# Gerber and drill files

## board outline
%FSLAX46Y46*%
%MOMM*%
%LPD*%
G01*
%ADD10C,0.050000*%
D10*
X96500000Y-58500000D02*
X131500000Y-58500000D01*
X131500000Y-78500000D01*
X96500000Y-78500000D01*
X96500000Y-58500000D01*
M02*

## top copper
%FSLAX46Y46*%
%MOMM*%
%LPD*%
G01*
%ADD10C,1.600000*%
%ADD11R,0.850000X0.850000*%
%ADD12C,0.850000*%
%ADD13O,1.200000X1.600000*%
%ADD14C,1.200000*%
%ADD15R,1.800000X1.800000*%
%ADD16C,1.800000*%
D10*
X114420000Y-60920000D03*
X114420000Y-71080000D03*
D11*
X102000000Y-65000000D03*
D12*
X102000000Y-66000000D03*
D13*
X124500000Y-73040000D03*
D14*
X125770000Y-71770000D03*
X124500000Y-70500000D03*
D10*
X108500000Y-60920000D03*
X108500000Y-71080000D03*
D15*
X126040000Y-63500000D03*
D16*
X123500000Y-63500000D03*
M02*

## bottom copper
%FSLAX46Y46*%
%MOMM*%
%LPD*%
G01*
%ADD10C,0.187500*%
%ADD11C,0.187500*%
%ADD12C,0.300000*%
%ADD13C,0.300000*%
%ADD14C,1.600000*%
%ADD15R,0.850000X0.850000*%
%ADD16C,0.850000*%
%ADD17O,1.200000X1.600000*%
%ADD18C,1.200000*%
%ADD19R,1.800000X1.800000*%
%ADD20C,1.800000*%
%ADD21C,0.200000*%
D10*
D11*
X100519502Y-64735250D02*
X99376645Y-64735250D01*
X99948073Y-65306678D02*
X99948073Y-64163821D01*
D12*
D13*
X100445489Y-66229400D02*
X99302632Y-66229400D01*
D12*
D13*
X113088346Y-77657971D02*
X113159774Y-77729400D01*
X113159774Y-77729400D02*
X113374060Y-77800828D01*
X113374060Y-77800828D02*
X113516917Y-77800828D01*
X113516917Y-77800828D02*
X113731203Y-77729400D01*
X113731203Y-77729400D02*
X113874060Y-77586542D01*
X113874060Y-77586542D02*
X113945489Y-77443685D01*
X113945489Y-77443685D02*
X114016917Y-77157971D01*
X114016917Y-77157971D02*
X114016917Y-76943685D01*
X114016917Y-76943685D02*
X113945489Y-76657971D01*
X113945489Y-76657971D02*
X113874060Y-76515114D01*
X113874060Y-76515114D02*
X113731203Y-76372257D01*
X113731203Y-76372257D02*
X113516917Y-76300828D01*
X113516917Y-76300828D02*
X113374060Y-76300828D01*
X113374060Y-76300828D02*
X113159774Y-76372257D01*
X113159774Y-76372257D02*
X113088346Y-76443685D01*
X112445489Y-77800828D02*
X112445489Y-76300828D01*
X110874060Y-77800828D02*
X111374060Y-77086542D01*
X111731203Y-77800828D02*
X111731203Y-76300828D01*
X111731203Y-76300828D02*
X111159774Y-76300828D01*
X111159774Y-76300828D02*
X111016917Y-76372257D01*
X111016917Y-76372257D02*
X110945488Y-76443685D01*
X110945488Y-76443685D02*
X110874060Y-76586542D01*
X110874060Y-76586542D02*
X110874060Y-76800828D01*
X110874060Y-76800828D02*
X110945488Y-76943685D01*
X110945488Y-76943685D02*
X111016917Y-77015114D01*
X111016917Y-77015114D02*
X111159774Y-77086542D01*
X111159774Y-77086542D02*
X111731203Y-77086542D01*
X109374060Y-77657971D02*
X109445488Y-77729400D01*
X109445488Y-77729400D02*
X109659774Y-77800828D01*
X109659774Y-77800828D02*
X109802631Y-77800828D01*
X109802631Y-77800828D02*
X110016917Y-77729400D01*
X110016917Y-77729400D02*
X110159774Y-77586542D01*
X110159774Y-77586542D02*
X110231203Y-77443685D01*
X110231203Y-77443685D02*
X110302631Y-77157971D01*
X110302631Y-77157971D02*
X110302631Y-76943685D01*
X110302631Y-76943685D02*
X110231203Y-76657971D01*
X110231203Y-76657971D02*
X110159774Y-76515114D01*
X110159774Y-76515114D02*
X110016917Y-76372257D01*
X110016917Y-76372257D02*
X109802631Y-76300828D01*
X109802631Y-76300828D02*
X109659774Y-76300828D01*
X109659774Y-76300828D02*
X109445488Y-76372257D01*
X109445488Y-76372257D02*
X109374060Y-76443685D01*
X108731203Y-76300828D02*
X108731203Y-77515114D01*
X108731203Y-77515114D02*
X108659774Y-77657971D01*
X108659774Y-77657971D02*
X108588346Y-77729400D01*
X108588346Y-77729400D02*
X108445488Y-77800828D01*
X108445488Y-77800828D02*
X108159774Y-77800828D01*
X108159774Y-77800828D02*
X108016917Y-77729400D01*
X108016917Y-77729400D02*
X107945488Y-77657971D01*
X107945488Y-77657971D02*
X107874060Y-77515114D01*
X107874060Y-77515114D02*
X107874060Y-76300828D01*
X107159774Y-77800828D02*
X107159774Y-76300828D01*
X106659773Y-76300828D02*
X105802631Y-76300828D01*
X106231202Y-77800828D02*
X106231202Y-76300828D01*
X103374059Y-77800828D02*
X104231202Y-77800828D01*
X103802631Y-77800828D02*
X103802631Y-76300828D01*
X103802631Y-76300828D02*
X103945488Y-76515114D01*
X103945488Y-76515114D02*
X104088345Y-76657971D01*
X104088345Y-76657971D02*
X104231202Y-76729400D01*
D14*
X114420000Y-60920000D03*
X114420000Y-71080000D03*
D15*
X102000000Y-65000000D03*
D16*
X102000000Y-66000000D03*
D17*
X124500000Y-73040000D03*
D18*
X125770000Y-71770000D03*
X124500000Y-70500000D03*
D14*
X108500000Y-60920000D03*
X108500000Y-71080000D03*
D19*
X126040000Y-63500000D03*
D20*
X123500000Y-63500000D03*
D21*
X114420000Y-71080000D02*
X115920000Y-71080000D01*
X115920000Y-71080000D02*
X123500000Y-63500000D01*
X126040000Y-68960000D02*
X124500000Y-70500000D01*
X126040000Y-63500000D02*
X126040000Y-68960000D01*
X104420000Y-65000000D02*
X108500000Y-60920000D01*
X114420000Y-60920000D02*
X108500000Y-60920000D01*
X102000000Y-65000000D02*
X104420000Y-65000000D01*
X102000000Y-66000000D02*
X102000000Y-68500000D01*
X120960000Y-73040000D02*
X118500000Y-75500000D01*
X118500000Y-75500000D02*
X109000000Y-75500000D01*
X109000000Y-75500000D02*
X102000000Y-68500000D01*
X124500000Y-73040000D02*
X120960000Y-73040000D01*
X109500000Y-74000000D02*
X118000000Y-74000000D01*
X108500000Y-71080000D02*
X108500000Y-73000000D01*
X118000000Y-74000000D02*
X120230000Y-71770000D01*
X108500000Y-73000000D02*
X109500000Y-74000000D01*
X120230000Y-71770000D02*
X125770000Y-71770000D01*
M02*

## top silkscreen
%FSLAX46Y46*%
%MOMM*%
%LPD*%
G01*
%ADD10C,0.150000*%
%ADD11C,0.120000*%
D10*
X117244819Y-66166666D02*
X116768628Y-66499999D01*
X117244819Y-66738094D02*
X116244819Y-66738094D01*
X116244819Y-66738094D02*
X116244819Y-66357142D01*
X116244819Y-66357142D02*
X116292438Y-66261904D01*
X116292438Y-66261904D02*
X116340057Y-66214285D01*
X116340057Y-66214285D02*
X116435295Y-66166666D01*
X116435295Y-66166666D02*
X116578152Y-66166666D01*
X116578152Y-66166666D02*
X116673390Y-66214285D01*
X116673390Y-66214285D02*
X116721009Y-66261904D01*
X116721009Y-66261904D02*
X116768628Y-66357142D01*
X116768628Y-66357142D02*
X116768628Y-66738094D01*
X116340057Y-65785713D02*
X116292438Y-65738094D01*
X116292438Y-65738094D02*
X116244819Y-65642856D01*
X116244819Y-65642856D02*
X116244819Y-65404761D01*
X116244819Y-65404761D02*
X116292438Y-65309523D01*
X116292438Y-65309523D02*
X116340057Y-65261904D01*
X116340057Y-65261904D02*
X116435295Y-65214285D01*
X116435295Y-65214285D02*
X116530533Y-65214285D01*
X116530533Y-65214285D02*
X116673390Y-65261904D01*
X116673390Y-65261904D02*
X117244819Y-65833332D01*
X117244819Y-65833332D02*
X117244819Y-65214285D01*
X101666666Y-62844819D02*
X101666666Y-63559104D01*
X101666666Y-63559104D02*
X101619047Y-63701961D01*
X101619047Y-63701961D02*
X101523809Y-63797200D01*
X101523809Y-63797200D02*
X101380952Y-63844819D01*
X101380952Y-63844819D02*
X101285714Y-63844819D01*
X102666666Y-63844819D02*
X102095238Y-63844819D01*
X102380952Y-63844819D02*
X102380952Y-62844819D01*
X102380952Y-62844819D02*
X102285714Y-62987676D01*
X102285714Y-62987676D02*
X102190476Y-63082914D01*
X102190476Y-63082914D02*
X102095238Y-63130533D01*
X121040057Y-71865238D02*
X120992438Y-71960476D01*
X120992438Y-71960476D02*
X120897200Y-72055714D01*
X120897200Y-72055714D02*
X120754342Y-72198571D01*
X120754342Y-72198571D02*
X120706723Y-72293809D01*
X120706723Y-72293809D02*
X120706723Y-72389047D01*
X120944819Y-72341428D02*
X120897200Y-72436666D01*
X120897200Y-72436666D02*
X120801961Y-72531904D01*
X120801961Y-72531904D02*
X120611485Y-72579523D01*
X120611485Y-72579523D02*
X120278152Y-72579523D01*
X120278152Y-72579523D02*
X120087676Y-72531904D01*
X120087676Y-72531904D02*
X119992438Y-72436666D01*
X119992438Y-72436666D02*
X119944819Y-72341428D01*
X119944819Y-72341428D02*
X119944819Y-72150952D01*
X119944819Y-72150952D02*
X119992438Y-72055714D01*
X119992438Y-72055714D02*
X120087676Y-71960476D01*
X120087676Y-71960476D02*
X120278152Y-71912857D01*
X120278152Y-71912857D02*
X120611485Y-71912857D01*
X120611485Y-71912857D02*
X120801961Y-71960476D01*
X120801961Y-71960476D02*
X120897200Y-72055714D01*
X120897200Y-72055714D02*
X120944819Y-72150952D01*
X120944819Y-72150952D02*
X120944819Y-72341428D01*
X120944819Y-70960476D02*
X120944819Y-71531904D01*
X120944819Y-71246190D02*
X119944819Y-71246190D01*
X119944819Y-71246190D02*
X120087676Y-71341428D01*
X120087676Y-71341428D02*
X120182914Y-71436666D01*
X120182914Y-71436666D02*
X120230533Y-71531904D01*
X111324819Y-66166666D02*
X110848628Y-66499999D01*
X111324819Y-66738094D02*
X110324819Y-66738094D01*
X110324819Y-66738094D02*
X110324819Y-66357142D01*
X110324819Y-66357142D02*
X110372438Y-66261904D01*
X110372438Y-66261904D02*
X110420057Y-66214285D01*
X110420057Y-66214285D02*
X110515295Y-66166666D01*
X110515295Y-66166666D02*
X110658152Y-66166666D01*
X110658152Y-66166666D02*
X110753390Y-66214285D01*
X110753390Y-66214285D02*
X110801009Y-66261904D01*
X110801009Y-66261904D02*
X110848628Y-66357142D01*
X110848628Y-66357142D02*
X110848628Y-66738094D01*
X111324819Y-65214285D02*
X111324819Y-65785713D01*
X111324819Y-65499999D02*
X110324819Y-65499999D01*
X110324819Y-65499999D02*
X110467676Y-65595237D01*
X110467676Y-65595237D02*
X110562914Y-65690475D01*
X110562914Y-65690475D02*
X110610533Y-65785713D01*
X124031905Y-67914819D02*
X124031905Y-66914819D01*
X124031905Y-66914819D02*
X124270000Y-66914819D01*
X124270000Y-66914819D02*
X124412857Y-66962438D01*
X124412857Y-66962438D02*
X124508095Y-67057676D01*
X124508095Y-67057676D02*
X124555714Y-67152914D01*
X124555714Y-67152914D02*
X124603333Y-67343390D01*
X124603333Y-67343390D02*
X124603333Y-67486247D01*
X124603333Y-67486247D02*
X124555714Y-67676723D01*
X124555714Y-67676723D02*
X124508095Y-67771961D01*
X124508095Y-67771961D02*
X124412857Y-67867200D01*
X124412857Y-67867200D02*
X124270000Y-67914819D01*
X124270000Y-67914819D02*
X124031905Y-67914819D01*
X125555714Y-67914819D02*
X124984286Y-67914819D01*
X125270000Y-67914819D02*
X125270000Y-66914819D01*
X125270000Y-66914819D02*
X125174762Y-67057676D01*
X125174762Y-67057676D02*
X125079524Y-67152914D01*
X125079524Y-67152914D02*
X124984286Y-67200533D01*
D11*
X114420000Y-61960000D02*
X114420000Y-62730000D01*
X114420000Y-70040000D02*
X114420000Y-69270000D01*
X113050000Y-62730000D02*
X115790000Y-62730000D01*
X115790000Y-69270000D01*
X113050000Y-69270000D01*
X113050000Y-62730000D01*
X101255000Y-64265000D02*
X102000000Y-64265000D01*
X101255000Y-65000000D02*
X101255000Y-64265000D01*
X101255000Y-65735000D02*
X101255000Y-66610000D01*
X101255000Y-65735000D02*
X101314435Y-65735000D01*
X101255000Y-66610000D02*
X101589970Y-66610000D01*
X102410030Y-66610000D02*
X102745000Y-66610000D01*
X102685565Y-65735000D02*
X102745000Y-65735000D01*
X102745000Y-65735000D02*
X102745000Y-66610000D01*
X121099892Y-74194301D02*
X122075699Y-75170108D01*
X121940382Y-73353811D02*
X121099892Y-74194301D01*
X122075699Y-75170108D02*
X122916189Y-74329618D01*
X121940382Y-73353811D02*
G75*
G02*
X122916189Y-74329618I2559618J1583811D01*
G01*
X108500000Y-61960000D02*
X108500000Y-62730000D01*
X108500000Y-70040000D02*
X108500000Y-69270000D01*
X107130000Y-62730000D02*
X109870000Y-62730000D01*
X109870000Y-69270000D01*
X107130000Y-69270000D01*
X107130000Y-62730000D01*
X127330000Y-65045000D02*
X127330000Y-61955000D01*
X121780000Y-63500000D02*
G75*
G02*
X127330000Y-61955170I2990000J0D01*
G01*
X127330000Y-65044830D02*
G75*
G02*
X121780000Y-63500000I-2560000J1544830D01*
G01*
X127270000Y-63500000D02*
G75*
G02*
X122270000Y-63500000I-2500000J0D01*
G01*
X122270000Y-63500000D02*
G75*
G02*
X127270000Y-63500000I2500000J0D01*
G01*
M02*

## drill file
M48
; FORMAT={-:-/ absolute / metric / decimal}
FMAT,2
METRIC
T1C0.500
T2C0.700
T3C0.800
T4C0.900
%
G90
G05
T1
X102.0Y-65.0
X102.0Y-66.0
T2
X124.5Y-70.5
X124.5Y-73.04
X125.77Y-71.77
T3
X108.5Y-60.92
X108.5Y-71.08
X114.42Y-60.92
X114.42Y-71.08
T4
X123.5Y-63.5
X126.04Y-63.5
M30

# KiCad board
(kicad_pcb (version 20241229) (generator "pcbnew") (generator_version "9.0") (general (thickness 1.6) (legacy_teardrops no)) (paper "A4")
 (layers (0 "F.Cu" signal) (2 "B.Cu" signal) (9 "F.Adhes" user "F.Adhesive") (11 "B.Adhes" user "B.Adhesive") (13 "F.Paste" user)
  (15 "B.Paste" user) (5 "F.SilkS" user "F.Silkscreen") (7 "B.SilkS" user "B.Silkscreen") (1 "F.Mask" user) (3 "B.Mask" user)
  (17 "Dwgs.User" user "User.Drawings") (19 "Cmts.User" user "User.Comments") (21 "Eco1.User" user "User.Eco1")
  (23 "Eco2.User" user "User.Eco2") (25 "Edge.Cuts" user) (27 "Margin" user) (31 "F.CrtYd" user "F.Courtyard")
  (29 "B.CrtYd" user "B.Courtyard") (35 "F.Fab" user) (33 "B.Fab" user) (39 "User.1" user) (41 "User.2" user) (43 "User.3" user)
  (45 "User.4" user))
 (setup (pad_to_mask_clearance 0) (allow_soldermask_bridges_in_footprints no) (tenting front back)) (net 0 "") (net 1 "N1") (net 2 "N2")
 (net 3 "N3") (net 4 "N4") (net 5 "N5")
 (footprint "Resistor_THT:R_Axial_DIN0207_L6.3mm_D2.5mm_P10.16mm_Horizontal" (layer "F.Cu") (at 114.42 60.92 -90)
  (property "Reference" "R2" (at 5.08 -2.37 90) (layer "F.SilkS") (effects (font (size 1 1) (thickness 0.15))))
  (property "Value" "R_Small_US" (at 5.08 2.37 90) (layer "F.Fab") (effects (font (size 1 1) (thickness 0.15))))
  (fp_line (start 1.04 0) (end 1.81 0) (stroke (width 0.12) (type solid)) (layer "F.SilkS"))
  (fp_line (start 9.12 0) (end 8.35 0) (stroke (width 0.12) (type solid)) (layer "F.SilkS"))
  (fp_rect (start 1.81 -1.37) (end 8.35 1.37) (stroke (width 0.12) (type solid)) (fill no) (layer "F.SilkS"))
  (pad "1" thru_hole circle (at 0 0 270) (size 1.6 1.6) (drill 0.8) (layers "*.Cu" "*.Mask") (remove_unused_layers no) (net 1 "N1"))
  (pad "2" thru_hole circle (at 10.16 0 270) (size 1.6 1.6) (drill 0.8) (layers "*.Cu" "*.Mask") (remove_unused_layers no) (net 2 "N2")))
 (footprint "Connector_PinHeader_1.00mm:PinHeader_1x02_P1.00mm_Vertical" (layer "F.Cu") (at 102 65)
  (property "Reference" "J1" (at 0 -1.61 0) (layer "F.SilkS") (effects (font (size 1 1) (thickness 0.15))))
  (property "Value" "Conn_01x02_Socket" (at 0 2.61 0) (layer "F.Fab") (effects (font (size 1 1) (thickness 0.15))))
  (fp_line (start -0.745 -0.735) (end 0 -0.735) (stroke (width 0.12) (type solid)) (layer "F.SilkS"))
  (fp_line (start -0.745 0) (end -0.745 -0.735) (stroke (width 0.12) (type solid)) (layer "F.SilkS"))
  (fp_line (start -0.745 0.735) (end -0.745 1.61) (stroke (width 0.12) (type solid)) (layer "F.SilkS"))
  (fp_line (start -0.745 0.735) (end -0.685565 0.735) (stroke (width 0.12) (type solid)) (layer "F.SilkS"))
  (fp_line (start -0.745 1.61) (end -0.41003 1.61) (stroke (width 0.12) (type solid)) (layer "F.SilkS"))
  (fp_line (start 0.41003 1.61) (end 0.745 1.61) (stroke (width 0.12) (type solid)) (layer "F.SilkS"))
  (fp_line (start 0.685565 0.735) (end 0.745 0.735) (stroke (width 0.12) (type solid)) (layer "F.SilkS"))
  (fp_line (start 0.745 0.735) (end 0.745 1.61) (stroke (width 0.12) (type solid)) (layer "F.SilkS"))
  (pad "1" thru_hole rect (at 0 0) (size 0.85 0.85) (drill 0.5) (layers "*.Cu" "*.Mask") (remove_unused_layers no) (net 1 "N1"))
  (pad "2" thru_hole circle (at 0 1) (size 0.85 0.85) (drill 0.5) (layers "*.Cu" "*.Mask") (remove_unused_layers no) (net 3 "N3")))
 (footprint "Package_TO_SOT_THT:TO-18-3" (layer "F.Cu") (at 124.5 73.04 90)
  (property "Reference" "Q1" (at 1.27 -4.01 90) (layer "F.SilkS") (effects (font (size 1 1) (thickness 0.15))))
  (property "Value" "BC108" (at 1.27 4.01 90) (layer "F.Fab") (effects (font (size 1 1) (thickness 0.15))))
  (fp_line (start -1.154301 -3.400108) (end -2.130108 -2.424301) (stroke (width 0.12) (type solid)) (layer "F.SilkS"))
  (fp_line (start -0.313811 -2.559618) (end -1.154301 -3.400108) (stroke (width 0.12) (type solid)) (layer "F.SilkS"))
  (fp_line (start -2.130108 -2.424301) (end -1.289618 -1.583811) (stroke (width 0.12) (type solid)) (layer "F.SilkS"))
  (fp_arc (start -0.313811 -2.559618) (mid 3.398391 2.128391) (end -1.289618 -1.583811) (stroke (width 0.12) (type solid)) (layer "F.SilkS"))
  (pad "1" thru_hole oval (at 0 0 90) (size 1.6 1.2) (drill 0.7) (layers "*.Cu" "*.Mask") (remove_unused_layers no) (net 3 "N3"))
  (pad "2" thru_hole circle (at 1.27 1.27 90) (size 1.2 1.2) (drill 0.7) (layers "*.Cu" "*.Mask") (remove_unused_layers no) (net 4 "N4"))
  (pad "3" thru_hole circle (at 2.54 0 90) (size 1.2 1.2) (drill 0.7) (layers "*.Cu" "*.Mask") (remove_unused_layers no) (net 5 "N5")))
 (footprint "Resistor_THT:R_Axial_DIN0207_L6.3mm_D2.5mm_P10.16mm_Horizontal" (layer "F.Cu") (at 108.5 60.92 -90)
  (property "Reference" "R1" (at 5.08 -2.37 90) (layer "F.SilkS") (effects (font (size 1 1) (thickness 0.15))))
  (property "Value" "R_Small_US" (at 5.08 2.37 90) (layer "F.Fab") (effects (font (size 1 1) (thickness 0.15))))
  (fp_line (start 1.04 0) (end 1.81 0) (stroke (width 0.12) (type solid)) (layer "F.SilkS"))
  (fp_line (start 9.12 0) (end 8.35 0) (stroke (width 0.12) (type solid)) (layer "F.SilkS"))
  (fp_rect (start 1.81 -1.37) (end 8.35 1.37) (stroke (width 0.12) (type solid)) (fill no) (layer "F.SilkS"))
  (pad "1" thru_hole circle (at 0 0 270) (size 1.6 1.6) (drill 0.8) (layers "*.Cu" "*.Mask") (remove_unused_layers no) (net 1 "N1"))
  (pad "2" thru_hole circle (at 10.16 0 270) (size 1.6 1.6) (drill 0.8) (layers "*.Cu" "*.Mask") (remove_unused_layers no) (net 4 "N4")))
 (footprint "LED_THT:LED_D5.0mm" (layer "F.Cu") (at 126.04 63.5 180)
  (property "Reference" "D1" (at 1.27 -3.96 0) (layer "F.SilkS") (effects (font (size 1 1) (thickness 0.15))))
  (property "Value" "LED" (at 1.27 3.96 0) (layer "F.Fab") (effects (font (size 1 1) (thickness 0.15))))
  (fp_line (start -1.29 -1.545) (end -1.29 1.545) (stroke (width 0.12) (type solid)) (layer "F.SilkS"))
  (fp_arc (start 4.26 0) (mid 2.071779 2.880495) (end -1.29 1.54483) (stroke (width 0.12) (type solid)) (layer "F.SilkS"))
  (fp_arc (start -1.29 -1.54483) (mid 2.071779 -2.880495) (end 4.26 0) (stroke (width 0.12) (type solid)) (layer "F.SilkS"))
  (fp_circle (center 1.27 0) (end 3.77 0) (stroke (width 0.12) (type solid)) (fill no) (layer "F.SilkS"))
  (pad "1" thru_hole rect (at 0 0 180) (size 1.8 1.8) (drill 0.9) (layers "*.Cu" "*.Mask") (remove_unused_layers no) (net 5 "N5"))
  (pad "2" thru_hole circle (at 2.54 0 180) (size 1.8 1.8) (drill 0.9) (layers "*.Cu" "*.Mask") (remove_unused_layers no) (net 2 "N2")))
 (gr_rect (start 96.5 58.5) (end 131.5 78.5) (stroke (width 0.05) (type solid)) (fill no) (layer "Edge.Cuts"))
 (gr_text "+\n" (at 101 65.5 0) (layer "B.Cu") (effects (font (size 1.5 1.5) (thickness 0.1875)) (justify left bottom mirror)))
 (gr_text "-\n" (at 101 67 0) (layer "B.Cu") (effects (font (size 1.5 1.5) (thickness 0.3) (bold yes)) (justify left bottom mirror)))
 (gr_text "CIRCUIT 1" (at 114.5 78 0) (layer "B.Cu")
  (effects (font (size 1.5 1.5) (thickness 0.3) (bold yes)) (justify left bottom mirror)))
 (segment (start 114.42 71.08) (end 115.92 71.08) (width 0.2) (layer "B.Cu") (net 2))
 (segment (start 115.92 71.08) (end 123.5 63.5) (width 0.2) (layer "B.Cu") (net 2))
 (segment (start 126.04 68.96) (end 124.5 70.5) (width 0.2) (layer "B.Cu") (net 5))
 (segment (start 126.04 63.5) (end 126.04 68.96) (width 0.2) (layer "B.Cu") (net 5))
 (segment (start 104.42 65) (end 108.5 60.92) (width 0.2) (layer "B.Cu") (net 1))
 (segment (start 114.42 60.92) (end 108.5 60.92) (width 0.2) (layer "B.Cu") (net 1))
 (segment (start 102 65) (end 104.42 65) (width 0.2) (layer "B.Cu") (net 1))
 (segment (start 102 66) (end 102 68.5) (width 0.2) (layer "B.Cu") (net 3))
 (segment (start 120.96 73.04) (end 118.5 75.5) (width 0.2) (layer "B.Cu") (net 3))
 (segment (start 118.5 75.5) (end 109 75.5) (width 0.2) (layer "B.Cu") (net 3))
 (segment (start 109 75.5) (end 102 68.5) (width 0.2) (layer "B.Cu") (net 3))
 (segment (start 124.5 73.04) (end 120.96 73.04) (width 0.2) (layer "B.Cu") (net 3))
 (segment (start 109.5 74) (end 118 74) (width 0.2) (layer "B.Cu") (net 4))
 (segment (start 108.5 71.08) (end 108.5 73) (width 0.2) (layer "B.Cu") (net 4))
 (segment (start 118 74) (end 120.23 71.77) (width 0.2) (layer "B.Cu") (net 4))
 (segment (start 108.5 73) (end 109.5 74) (width 0.2) (layer "B.Cu") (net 4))
 (segment (start 120.23 71.77) (end 125.77 71.77) (width 0.2) (layer "B.Cu") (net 4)))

